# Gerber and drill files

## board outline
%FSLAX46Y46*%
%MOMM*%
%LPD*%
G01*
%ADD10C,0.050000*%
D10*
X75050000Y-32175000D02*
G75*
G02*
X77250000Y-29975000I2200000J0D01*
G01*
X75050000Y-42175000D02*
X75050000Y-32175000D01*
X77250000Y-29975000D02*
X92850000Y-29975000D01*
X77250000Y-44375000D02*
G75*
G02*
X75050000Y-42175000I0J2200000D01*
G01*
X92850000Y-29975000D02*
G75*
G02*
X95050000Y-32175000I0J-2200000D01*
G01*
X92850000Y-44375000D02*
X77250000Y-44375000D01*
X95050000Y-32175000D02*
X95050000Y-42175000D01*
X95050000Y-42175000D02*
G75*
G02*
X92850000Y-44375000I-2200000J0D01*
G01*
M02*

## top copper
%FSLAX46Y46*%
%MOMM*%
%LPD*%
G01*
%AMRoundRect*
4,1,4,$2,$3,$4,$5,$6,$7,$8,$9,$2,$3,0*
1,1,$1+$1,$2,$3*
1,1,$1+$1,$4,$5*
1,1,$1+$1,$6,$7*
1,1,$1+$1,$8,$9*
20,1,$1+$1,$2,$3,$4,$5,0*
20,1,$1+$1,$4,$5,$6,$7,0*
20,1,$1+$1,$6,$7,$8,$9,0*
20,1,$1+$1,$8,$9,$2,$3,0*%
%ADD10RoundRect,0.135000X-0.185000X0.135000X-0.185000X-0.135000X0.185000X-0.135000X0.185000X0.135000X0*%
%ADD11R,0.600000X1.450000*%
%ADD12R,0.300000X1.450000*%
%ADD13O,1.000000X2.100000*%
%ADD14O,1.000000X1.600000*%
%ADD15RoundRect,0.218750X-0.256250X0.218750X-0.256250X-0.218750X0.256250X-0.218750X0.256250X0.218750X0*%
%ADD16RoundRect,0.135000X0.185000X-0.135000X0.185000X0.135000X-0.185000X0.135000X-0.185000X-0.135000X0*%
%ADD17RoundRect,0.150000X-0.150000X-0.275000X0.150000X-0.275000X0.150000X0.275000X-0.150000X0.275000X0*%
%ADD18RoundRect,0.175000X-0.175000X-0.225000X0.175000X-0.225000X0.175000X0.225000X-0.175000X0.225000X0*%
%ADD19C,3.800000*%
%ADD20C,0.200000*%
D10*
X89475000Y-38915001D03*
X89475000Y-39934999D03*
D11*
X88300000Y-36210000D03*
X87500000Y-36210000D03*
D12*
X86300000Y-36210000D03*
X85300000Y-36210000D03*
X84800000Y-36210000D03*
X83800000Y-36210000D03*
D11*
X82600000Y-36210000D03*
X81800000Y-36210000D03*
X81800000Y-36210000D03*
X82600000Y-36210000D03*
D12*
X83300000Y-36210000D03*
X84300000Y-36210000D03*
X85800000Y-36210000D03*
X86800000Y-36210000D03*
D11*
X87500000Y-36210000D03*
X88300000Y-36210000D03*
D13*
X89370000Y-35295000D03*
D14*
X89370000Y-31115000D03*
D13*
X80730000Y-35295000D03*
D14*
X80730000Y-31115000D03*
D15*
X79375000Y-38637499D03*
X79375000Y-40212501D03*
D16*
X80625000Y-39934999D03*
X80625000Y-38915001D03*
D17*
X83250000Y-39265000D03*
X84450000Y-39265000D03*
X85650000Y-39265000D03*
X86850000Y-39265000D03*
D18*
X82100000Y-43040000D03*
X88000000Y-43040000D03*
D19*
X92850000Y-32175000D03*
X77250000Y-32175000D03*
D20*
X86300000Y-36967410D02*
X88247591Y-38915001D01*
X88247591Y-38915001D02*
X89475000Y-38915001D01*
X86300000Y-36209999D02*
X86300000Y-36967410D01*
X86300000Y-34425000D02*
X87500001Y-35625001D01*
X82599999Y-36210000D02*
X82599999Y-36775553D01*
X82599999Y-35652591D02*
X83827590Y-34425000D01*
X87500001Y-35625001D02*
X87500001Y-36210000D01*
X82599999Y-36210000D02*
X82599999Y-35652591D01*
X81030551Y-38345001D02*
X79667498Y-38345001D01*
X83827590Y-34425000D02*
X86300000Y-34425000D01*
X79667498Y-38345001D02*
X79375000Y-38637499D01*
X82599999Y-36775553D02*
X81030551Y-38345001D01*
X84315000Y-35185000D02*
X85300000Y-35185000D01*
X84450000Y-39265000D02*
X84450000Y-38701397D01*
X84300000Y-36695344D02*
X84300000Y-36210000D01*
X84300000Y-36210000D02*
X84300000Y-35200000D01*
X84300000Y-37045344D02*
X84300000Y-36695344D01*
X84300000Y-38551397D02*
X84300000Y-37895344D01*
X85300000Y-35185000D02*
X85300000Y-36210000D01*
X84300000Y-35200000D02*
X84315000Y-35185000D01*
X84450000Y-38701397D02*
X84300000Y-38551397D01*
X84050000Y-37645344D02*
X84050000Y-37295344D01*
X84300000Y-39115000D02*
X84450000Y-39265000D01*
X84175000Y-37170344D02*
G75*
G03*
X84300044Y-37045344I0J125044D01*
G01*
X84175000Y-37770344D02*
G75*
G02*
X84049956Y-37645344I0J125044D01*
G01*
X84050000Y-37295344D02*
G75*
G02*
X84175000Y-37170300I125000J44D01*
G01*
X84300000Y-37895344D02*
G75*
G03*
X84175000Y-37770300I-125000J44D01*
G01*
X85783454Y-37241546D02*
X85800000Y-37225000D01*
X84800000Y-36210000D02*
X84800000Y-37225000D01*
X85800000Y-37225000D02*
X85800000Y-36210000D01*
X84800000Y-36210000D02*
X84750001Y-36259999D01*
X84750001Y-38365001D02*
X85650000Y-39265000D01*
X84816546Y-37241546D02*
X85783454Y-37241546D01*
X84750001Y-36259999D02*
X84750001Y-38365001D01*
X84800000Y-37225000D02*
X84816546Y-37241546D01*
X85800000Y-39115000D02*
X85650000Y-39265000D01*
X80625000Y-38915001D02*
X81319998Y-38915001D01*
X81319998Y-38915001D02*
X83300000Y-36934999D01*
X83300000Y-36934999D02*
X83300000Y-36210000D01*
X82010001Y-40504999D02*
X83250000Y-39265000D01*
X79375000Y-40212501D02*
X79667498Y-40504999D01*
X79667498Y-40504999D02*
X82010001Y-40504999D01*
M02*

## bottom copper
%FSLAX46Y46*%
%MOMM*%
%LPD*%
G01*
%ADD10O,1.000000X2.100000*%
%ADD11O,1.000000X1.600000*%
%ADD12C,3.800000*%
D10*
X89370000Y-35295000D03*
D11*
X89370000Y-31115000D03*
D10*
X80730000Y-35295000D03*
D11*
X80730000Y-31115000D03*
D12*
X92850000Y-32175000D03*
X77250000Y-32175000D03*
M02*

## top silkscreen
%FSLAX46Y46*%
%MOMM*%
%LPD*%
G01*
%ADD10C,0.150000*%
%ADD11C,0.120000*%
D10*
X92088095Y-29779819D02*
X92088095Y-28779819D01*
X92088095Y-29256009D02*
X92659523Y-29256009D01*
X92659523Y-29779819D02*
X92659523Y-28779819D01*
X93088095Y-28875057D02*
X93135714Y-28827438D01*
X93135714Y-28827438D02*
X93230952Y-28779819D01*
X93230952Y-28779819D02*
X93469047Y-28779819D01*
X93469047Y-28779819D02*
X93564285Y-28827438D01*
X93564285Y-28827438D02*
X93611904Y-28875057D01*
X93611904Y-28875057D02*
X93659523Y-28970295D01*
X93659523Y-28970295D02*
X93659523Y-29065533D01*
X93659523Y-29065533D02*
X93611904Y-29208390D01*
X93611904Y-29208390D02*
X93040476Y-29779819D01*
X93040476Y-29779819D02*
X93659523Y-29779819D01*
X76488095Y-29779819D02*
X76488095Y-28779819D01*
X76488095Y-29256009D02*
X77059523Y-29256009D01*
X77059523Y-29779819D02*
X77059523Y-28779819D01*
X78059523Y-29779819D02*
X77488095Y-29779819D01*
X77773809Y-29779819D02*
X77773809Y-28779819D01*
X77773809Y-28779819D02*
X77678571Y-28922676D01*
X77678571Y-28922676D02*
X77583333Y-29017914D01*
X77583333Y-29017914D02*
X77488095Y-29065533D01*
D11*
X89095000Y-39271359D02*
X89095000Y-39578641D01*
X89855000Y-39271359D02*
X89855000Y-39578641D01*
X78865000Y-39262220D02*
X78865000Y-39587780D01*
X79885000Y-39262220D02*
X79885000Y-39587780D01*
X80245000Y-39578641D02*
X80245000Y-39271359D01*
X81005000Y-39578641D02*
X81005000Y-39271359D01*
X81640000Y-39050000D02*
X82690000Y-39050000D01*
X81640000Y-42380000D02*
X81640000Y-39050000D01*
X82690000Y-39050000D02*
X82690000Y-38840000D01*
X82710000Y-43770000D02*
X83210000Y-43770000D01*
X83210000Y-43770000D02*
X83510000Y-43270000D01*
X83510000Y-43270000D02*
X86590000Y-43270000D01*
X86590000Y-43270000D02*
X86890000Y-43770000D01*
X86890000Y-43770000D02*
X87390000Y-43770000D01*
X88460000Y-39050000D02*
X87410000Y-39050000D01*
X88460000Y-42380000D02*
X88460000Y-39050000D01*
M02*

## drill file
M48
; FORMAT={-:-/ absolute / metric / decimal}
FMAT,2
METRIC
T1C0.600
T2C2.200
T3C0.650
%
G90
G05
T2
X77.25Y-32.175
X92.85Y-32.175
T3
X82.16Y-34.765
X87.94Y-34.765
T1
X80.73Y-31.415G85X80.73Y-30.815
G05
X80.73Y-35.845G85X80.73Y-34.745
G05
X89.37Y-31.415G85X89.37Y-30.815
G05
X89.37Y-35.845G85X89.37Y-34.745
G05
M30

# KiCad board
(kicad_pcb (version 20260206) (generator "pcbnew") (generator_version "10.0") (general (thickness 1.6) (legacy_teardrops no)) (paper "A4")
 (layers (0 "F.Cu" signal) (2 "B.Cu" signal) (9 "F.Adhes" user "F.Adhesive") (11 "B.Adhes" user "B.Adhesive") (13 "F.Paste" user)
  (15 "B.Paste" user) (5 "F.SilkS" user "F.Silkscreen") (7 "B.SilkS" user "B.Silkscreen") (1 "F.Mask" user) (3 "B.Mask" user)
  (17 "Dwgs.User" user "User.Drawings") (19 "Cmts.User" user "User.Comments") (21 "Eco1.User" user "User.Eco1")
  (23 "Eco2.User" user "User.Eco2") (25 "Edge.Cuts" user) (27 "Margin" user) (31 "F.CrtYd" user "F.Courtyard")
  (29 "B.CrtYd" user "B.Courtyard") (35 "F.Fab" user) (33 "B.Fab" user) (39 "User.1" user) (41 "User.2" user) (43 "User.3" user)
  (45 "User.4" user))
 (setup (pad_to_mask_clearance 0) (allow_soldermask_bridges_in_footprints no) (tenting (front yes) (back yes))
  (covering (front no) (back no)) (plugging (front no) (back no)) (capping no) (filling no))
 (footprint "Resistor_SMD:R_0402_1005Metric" (layer "F.Cu") (at 89.475 39.425 -90)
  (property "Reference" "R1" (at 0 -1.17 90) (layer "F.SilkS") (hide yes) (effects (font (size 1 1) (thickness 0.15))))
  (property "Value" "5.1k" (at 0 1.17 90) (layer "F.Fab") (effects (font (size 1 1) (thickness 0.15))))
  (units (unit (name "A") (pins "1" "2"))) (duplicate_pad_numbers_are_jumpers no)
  (fp_line (start -0.153641 0.38) (end 0.153641 0.38) (stroke (width 0.12) (type solid)) (layer "F.SilkS"))
  (fp_line (start -0.153641 -0.38) (end 0.153641 -0.38) (stroke (width 0.12) (type solid)) (layer "F.SilkS"))
  (pad "1" smd roundrect (at -0.509999 0 270) (size 0.54 0.64) (layers "F.Cu" "F.Mask" "F.Paste") (roundrect_rratio 0.25)
   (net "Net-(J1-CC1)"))
  (pad "2" smd roundrect (at 0.509999 0 270) (size 0.54 0.64) (layers "F.Cu" "F.Mask" "F.Paste") (roundrect_rratio 0.25) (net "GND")))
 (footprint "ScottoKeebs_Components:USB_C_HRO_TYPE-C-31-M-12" (layer "F.Cu") (at 85.05 32.165 180)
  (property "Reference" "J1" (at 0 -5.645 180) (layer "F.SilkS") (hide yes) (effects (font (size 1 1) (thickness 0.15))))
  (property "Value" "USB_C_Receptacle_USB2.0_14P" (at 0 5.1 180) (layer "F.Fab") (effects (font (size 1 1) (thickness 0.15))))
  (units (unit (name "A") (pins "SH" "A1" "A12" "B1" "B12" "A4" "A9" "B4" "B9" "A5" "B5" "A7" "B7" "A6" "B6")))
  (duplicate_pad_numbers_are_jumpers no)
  (pad "" np_thru_hole circle (at -2.89 -2.6 180) (size 0.65 0.65) (drill 0.65) (layers "*.Cu" "*.Mask"))
  (pad "" np_thru_hole circle (at 2.89 -2.6 180) (size 0.65 0.65) (drill 0.65) (layers "*.Cu" "*.Mask"))
  (pad "A1" smd rect (at -3.25 -4.045 180) (size 0.6 1.45) (layers "F.Cu" "F.Mask" "F.Paste") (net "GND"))
  (pad "A4" smd rect (at -2.45 -4.045 180) (size 0.6 1.45) (layers "F.Cu" "F.Mask" "F.Paste") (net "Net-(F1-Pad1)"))
  (pad "A5" smd rect (at -1.25 -4.045 180) (size 0.3 1.45) (layers "F.Cu" "F.Mask" "F.Paste") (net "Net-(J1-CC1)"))
  (pad "A6" smd rect (at -0.25 -4.045 180) (size 0.3 1.45) (layers "F.Cu" "F.Mask" "F.Paste") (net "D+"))
  (pad "A7" smd rect (at 0.25 -4.045 180) (size 0.3 1.45) (layers "F.Cu" "F.Mask" "F.Paste") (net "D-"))
  (pad "A8" smd rect (at 1.25 -4.045 180) (size 0.3 1.45) (layers "F.Cu" "F.Mask" "F.Paste"))
  (pad "A9" smd rect (at 2.45 -4.045 180) (size 0.6 1.45) (layers "F.Cu" "F.Mask" "F.Paste") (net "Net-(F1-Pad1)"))
  (pad "A12" smd rect (at 3.25 -4.045 180) (size 0.6 1.45) (layers "F.Cu" "F.Mask" "F.Paste") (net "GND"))
  (pad "B1" smd rect (at 3.25 -4.045 180) (size 0.6 1.45) (layers "F.Cu" "F.Mask" "F.Paste") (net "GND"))
  (pad "B4" smd rect (at 2.45 -4.045 180) (size 0.6 1.45) (layers "F.Cu" "F.Mask" "F.Paste") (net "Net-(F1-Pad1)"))
  (pad "B5" smd rect (at 1.75 -4.045 180) (size 0.3 1.45) (layers "F.Cu" "F.Mask" "F.Paste") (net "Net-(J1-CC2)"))
  (pad "B6" smd rect (at 0.75 -4.045 180) (size 0.3 1.45) (layers "F.Cu" "F.Mask" "F.Paste") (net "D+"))
  (pad "B7" smd rect (at -0.75 -4.045 180) (size 0.3 1.45) (layers "F.Cu" "F.Mask" "F.Paste") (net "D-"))
  (pad "B8" smd rect (at -1.75 -4.045 180) (size 0.3 1.45) (layers "F.Cu" "F.Mask" "F.Paste"))
  (pad "B9" smd rect (at -2.45 -4.045 180) (size 0.6 1.45) (layers "F.Cu" "F.Mask" "F.Paste") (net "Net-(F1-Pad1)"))
  (pad "B12" smd rect (at -3.25 -4.045 180) (size 0.6 1.45) (layers "F.Cu" "F.Mask" "F.Paste") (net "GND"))
  (pad "S1" thru_hole oval (at -4.32 -3.13 180) (size 1 2.1) (drill oval 0.6 1.7) (layers "*.Cu" "*.Mask") (remove_unused_layers no))
  (pad "S1" thru_hole oval (at -4.32 1.05 180) (size 1 1.6) (drill oval 0.6 1.2) (layers "*.Cu" "*.Mask") (remove_unused_layers no))
  (pad "S1" thru_hole oval (at 4.32 -3.13 180) (size 1 2.1) (drill oval 0.6 1.7) (layers "*.Cu" "*.Mask") (remove_unused_layers no))
  (pad "S1" thru_hole oval (at 4.32 1.05 180) (size 1 1.6) (drill oval 0.6 1.2) (layers "*.Cu" "*.Mask") (remove_unused_layers no)))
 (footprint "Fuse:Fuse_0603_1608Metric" (layer "F.Cu") (at 79.375 39.425 -90)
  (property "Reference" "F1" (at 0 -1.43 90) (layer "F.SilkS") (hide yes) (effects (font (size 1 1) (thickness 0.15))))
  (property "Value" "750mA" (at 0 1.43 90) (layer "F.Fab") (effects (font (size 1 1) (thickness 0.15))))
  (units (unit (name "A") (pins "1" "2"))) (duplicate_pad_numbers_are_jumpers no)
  (fp_line (start -0.16278 0.51) (end 0.16278 0.51) (stroke (width 0.12) (type solid)) (layer "F.SilkS"))
  (fp_line (start -0.16278 -0.51) (end 0.16278 -0.51) (stroke (width 0.12) (type solid)) (layer "F.SilkS"))
  (pad "1" smd roundrect (at -0.787501 0 270) (size 0.875 0.95) (layers "F.Cu" "F.Mask" "F.Paste") (roundrect_rratio 0.25)
   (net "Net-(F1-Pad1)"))
  (pad "2" smd roundrect (at 0.787501 0 270) (size 0.875 0.95) (layers "F.Cu" "F.Mask" "F.Paste") (roundrect_rratio 0.25) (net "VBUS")))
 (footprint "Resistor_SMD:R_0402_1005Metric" (layer "F.Cu") (at 80.625 39.425 90)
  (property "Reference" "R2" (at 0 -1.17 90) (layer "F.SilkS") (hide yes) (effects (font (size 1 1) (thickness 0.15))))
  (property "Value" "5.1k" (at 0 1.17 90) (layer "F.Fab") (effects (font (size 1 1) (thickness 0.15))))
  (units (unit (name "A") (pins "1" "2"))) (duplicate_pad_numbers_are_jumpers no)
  (fp_line (start -0.153641 -0.38) (end 0.153641 -0.38) (stroke (width 0.12) (type solid)) (layer "F.SilkS"))
  (fp_line (start -0.153641 0.38) (end 0.153641 0.38) (stroke (width 0.12) (type solid)) (layer "F.SilkS"))
  (pad "1" smd roundrect (at -0.509999 0 90) (size 0.54 0.64) (layers "F.Cu" "F.Mask" "F.Paste") (roundrect_rratio 0.25) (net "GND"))
  (pad "2" smd roundrect (at 0.509999 0 90) (size 0.54 0.64) (layers "F.Cu" "F.Mask" "F.Paste") (roundrect_rratio 0.25) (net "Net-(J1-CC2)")))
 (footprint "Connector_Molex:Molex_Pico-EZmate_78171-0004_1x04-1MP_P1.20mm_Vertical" (layer "F.Cu") (at 85.05 41.14)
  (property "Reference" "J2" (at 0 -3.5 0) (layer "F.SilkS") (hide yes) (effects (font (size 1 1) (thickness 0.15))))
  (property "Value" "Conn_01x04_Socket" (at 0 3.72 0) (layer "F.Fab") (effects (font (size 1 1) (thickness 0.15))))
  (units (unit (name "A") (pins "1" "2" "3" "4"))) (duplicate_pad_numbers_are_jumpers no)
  (fp_line (start -3.41 -2.09) (end -2.36 -2.09) (stroke (width 0.12) (type solid)) (layer "F.SilkS"))
  (fp_line (start -3.41 1.24) (end -3.41 -2.09) (stroke (width 0.12) (type solid)) (layer "F.SilkS"))
  (fp_line (start -2.36 -2.09) (end -2.36 -2.3) (stroke (width 0.12) (type solid)) (layer "F.SilkS"))
  (fp_line (start -2.34 2.63) (end -1.84 2.63) (stroke (width 0.12) (type solid)) (layer "F.SilkS"))
  (fp_line (start -1.84 2.63) (end -1.54 2.13) (stroke (width 0.12) (type solid)) (layer "F.SilkS"))
  (fp_line (start -1.54 2.13) (end 1.54 2.13) (stroke (width 0.12) (type solid)) (layer "F.SilkS"))
  (fp_line (start 1.54 2.13) (end 1.84 2.63) (stroke (width 0.12) (type solid)) (layer "F.SilkS"))
  (fp_line (start 1.84 2.63) (end 2.34 2.63) (stroke (width 0.12) (type solid)) (layer "F.SilkS"))
  (fp_line (start 3.41 -2.09) (end 2.36 -2.09) (stroke (width 0.12) (type solid)) (layer "F.SilkS"))
  (fp_line (start 3.41 1.24) (end 3.41 -2.09) (stroke (width 0.12) (type solid)) (layer "F.SilkS"))
  (pad "1" smd roundrect (at -1.8 -1.875) (size 0.6 0.85) (layers "F.Cu" "F.Mask" "F.Paste") (roundrect_rratio 0.25) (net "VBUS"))
  (pad "2" smd roundrect (at -0.6 -1.875) (size 0.6 0.85) (layers "F.Cu" "F.Mask" "F.Paste") (roundrect_rratio 0.25) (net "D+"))
  (pad "3" smd roundrect (at 0.6 -1.875) (size 0.6 0.85) (layers "F.Cu" "F.Mask" "F.Paste") (roundrect_rratio 0.25) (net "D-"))
  (pad "4" smd roundrect (at 1.8 -1.875) (size 0.6 0.85) (layers "F.Cu" "F.Mask" "F.Paste") (roundrect_rratio 0.25) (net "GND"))
  (pad "MP" smd roundrect (at -2.95 1.9) (size 0.7 0.8) (layers "F.Cu" "F.Mask" "F.Paste") (roundrect_rratio 0.25))
  (pad "MP" smd roundrect (at 2.95 1.9) (size 0.7 0.8) (layers "F.Cu" "F.Mask" "F.Paste") (roundrect_rratio 0.25)))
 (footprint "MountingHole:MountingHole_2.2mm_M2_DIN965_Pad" (layer "F.Cu") (at 92.85 32.175)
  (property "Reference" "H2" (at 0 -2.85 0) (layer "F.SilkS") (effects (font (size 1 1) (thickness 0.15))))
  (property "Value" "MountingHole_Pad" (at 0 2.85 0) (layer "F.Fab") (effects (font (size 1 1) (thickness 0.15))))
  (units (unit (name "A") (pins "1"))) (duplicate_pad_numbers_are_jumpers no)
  (pad "1" thru_hole circle (at 0 0) (size 3.8 3.8) (drill 2.2) (layers "*.Cu" "*.Mask") (remove_unused_layers no) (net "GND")
   (zone_connect 2)))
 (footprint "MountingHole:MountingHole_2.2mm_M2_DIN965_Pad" (layer "F.Cu") (at 77.25 32.175)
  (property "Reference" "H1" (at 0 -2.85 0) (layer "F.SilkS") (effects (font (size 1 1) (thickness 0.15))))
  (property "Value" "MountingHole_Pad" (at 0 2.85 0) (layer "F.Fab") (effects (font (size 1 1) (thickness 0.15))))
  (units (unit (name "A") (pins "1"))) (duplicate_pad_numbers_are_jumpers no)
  (pad "1" thru_hole circle (at 0 0) (size 3.8 3.8) (drill 2.2) (layers "*.Cu" "*.Mask") (remove_unused_layers no) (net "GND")
   (zone_connect 2)))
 (gr_arc (start 75.05 32.175) (mid 75.694365 30.619365) (end 77.25 29.975) (stroke (width 0.05) (type default)) (layer "Edge.Cuts"))
 (gr_line (start 75.05 42.175) (end 75.05 32.175) (stroke (width 0.05) (type solid)) (layer "Edge.Cuts"))
 (gr_line (start 77.25 29.975) (end 92.85 29.975) (stroke (width 0.05) (type default)) (layer "Edge.Cuts"))
 (gr_arc (start 77.25 44.375) (mid 75.694365 43.730635) (end 75.05 42.175) (stroke (width 0.05) (type default)) (layer "Edge.Cuts"))
 (gr_arc (start 92.85 29.975) (mid 94.405635 30.619365) (end 95.05 32.175) (stroke (width 0.05) (type default)) (layer "Edge.Cuts"))
 (gr_line (start 92.85 44.375) (end 77.25 44.375) (stroke (width 0.05) (type default)) (layer "Edge.Cuts"))
 (gr_line (start 95.05 32.175) (end 95.05 42.175) (stroke (width 0.05) (type default)) (layer "Edge.Cuts"))
 (gr_arc (start 95.05 42.175) (mid 94.405635 43.730635) (end 92.85 44.375) (stroke (width 0.05) (type default)) (layer "Edge.Cuts"))
 (segment (start 86.3 36.96741) (end 88.247591 38.915001) (width 0.2) (layer "F.Cu") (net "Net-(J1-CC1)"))
 (segment (start 88.247591 38.915001) (end 89.475 38.915001) (width 0.2) (layer "F.Cu") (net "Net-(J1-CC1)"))
 (segment (start 86.3 36.209999) (end 86.3 36.96741) (width 0.2) (layer "F.Cu") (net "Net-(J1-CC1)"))
 (segment (start 86.3 34.425) (end 87.500001 35.625001) (width 0.2) (layer "F.Cu") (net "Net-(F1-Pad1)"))
 (segment (start 82.599999 36.21) (end 82.599999 36.775553) (width 0.2) (layer "F.Cu") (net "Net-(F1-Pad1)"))
 (segment (start 82.599999 35.652591) (end 83.82759 34.425) (width 0.2) (layer "F.Cu") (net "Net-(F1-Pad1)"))
 (segment (start 87.500001 35.625001) (end 87.500001 36.21) (width 0.2) (layer "F.Cu") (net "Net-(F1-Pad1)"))
 (segment (start 82.599999 36.21) (end 82.599999 35.652591) (width 0.2) (layer "F.Cu") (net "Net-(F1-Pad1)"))
 (segment (start 81.030551 38.345001) (end 79.667498 38.345001) (width 0.2) (layer "F.Cu") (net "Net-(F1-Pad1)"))
 (segment (start 83.82759 34.425) (end 86.3 34.425) (width 0.2) (layer "F.Cu") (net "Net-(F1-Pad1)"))
 (segment (start 79.667498 38.345001) (end 79.375 38.637499) (width 0.2) (layer "F.Cu") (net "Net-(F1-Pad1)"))
 (segment (start 82.599999 36.775553) (end 81.030551 38.345001) (width 0.2) (layer "F.Cu") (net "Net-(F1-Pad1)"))
 (segment (start 84.315 35.185) (end 85.3 35.185) (width 0.2) (layer "F.Cu") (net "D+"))
 (segment (start 84.45 39.265) (end 84.45 38.701397) (width 0.2) (layer "F.Cu") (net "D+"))
 (segment (start 84.3 36.695344) (end 84.3 36.21) (width 0.2) (layer "F.Cu") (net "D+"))
 (segment (start 84.3 36.21) (end 84.3 35.2) (width 0.2) (layer "F.Cu") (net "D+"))
 (segment (start 84.3 37.045344) (end 84.3 36.695344) (width 0.2) (layer "F.Cu") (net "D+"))
 (segment (start 84.3 38.551397) (end 84.3 37.895344) (width 0.2) (layer "F.Cu") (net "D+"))
 (segment (start 85.3 35.185) (end 85.3 36.21) (width 0.2) (layer "F.Cu") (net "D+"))
 (segment (start 84.3 35.2) (end 84.315 35.185) (width 0.2) (layer "F.Cu") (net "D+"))
 (segment (start 84.45 38.701397) (end 84.3 38.551397) (width 0.2) (layer "F.Cu") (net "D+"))
 (segment (start 84.05 37.645344) (end 84.05 37.295344) (width 0.2) (layer "F.Cu") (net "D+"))
 (segment (start 84.3 39.115) (end 84.45 39.265) (width 0.2) (layer "F.Cu") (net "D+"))
 (arc (start 84.175 37.170344) (mid 84.263388 37.133732) (end 84.3 37.045344) (width 0.2) (layer "F.Cu") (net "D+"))
 (arc (start 84.175 37.770344) (mid 84.086612 37.733732) (end 84.05 37.645344) (width 0.2) (layer "F.Cu") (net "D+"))
 (arc (start 84.05 37.295344) (mid 84.086612 37.206956) (end 84.175 37.170344) (width 0.2) (layer "F.Cu") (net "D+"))
 (arc (start 84.3 37.895344) (mid 84.263388 37.806956) (end 84.175 37.770344) (width 0.2) (layer "F.Cu") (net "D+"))
 (segment (start 85.783454 37.241546) (end 85.8 37.225) (width 0.2) (layer "F.Cu") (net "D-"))
 (segment (start 84.8 36.21) (end 84.8 37.225) (width 0.2) (layer "F.Cu") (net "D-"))
 (segment (start 85.8 37.225) (end 85.8 36.21) (width 0.2) (layer "F.Cu") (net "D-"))
 (segment (start 84.8 36.21) (end 84.750001 36.259999) (width 0.2) (layer "F.Cu") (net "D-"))
 (segment (start 84.750001 38.365001) (end 85.65 39.265) (width 0.2) (layer "F.Cu") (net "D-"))
 (segment (start 84.816546 37.241546) (end 85.783454 37.241546) (width 0.2) (layer "F.Cu") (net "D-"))
 (segment (start 84.750001 36.259999) (end 84.750001 38.365001) (width 0.2) (layer "F.Cu") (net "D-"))
 (segment (start 84.8 37.225) (end 84.816546 37.241546) (width 0.2) (layer "F.Cu") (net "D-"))
 (segment (start 85.8 39.115) (end 85.65 39.265) (width 0.2) (layer "F.Cu") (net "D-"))
 (segment (start 80.625 38.915001) (end 81.319998 38.915001) (width 0.2) (layer "F.Cu") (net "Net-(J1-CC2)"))
 (segment (start 81.319998 38.915001) (end 83.3 36.934999) (width 0.2) (layer "F.Cu") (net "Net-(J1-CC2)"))
 (segment (start 83.3 36.934999) (end 83.3 36.21) (width 0.2) (layer "F.Cu") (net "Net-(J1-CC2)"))
 (segment (start 82.010001 40.504999) (end 83.25 39.265) (width 0.2) (layer "F.Cu") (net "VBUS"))
 (segment (start 79.375 40.212501) (end 79.667498 40.504999) (width 0.2) (layer "F.Cu") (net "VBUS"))
 (segment (start 79.667498 40.504999) (end 82.010001 40.504999) (width 0.2) (layer "F.Cu") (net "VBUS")))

